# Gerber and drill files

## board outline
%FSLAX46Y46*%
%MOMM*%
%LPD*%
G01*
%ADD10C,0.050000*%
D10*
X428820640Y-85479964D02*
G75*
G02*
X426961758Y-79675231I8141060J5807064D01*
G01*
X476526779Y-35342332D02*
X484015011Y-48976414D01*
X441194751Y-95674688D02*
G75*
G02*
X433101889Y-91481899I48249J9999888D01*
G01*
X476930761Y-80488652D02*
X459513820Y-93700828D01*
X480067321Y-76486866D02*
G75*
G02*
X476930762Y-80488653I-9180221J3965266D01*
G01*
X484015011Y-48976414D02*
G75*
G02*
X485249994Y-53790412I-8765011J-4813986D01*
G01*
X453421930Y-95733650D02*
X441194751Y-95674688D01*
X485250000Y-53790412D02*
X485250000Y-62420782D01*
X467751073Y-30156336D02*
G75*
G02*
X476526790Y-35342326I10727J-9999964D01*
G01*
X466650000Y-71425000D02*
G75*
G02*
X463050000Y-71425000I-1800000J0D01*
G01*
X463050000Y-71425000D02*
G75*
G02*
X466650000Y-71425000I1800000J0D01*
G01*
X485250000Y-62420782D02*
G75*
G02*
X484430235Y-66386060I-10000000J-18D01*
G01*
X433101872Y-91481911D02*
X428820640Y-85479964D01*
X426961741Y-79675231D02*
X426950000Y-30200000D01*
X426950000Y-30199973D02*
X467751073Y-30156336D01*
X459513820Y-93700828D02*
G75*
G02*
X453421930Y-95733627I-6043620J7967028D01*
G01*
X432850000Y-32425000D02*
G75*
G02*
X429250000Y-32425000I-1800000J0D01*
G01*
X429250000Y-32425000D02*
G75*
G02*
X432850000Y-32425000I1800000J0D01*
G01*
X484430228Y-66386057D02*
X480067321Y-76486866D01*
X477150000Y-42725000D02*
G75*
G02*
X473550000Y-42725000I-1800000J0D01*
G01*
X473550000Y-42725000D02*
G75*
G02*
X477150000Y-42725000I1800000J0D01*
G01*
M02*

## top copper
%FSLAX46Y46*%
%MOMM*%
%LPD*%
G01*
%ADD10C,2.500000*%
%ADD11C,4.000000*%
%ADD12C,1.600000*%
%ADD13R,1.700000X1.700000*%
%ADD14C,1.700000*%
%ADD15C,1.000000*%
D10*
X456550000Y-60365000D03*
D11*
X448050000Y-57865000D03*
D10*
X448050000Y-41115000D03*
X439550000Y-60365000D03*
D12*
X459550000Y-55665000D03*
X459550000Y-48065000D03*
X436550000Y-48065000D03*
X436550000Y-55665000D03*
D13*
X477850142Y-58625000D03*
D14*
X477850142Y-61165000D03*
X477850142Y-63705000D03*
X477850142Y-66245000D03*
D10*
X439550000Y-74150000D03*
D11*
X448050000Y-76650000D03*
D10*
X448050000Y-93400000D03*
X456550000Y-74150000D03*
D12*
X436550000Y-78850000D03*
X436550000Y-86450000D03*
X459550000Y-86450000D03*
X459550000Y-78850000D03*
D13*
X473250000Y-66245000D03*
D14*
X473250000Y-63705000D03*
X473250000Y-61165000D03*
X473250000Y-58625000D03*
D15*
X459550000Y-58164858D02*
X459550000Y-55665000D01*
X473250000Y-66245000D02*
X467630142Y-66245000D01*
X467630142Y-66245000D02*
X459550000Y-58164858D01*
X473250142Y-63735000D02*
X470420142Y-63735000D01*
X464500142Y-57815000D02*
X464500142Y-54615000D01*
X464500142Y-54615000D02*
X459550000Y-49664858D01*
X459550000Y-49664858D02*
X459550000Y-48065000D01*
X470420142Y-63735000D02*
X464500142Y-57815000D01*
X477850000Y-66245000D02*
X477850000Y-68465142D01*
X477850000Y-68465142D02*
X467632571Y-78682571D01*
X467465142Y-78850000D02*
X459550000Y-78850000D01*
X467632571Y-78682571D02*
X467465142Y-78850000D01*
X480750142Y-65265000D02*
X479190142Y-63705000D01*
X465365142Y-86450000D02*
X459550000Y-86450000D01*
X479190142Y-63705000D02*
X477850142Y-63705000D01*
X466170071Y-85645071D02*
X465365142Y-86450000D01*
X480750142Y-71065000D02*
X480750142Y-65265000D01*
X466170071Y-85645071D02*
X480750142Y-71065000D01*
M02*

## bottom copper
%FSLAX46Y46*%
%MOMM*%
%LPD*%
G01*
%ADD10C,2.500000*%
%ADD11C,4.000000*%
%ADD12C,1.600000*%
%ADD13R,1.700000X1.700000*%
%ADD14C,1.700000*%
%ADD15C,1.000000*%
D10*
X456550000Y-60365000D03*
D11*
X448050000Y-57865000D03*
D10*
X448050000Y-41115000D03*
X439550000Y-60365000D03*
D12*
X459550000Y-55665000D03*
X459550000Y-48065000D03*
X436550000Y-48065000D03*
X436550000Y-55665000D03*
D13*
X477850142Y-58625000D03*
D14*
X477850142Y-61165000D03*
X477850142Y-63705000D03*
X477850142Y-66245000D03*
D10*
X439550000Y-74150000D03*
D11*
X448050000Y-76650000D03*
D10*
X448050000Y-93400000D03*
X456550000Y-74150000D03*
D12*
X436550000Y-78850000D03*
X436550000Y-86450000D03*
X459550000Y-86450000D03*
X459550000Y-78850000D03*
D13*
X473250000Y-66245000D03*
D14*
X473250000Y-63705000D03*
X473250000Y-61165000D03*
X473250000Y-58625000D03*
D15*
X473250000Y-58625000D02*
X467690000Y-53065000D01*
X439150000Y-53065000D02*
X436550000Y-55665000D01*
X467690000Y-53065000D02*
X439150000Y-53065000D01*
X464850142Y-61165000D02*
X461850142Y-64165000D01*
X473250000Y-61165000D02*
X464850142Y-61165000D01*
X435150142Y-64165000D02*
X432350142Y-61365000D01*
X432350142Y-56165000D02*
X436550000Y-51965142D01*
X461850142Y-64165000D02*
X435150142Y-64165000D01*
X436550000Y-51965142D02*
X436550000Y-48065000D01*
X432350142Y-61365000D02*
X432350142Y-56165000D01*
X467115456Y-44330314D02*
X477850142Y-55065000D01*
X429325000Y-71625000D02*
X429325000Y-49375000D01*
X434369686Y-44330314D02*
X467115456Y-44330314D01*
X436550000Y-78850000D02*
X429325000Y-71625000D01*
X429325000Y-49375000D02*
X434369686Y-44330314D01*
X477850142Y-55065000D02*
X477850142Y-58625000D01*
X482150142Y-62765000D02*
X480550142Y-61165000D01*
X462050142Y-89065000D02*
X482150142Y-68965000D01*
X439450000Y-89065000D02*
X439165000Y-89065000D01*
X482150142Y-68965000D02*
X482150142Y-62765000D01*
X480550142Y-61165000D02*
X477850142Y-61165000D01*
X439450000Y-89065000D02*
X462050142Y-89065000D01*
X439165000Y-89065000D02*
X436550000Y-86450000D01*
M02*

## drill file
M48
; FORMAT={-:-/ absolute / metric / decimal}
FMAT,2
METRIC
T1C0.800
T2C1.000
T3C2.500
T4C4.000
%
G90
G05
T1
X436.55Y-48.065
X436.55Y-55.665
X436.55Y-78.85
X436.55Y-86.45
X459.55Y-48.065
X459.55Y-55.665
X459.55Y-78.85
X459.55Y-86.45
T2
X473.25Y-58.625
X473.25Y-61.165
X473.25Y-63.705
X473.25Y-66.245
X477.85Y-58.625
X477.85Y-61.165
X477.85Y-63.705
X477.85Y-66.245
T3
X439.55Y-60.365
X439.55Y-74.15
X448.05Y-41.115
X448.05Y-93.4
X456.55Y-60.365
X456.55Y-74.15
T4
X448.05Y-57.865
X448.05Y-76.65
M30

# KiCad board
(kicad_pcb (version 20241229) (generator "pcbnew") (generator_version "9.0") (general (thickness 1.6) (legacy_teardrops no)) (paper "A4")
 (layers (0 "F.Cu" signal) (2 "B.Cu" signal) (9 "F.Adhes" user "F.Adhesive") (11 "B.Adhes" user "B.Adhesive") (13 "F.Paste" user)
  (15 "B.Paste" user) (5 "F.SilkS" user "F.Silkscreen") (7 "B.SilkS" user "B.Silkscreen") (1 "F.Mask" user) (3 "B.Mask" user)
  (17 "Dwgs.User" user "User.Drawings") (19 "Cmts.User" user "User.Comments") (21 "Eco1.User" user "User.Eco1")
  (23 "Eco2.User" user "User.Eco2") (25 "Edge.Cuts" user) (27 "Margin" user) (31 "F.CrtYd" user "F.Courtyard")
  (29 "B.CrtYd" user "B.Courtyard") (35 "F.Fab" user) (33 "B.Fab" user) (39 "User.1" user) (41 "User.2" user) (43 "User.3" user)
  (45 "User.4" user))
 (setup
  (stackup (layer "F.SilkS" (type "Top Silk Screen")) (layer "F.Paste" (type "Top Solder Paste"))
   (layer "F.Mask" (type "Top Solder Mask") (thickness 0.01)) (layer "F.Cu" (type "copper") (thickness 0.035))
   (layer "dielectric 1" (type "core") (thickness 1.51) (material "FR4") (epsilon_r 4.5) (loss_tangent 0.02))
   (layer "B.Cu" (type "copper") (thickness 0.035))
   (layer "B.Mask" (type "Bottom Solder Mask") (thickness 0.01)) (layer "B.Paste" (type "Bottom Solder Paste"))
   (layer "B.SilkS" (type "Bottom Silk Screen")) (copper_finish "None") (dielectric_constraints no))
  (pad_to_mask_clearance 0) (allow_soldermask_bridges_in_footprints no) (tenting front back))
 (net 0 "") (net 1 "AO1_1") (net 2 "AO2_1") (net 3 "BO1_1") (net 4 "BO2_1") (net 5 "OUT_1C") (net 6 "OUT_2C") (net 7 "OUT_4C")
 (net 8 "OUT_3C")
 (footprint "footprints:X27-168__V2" (layer "F.Cu") (at 448.05 51.865 180)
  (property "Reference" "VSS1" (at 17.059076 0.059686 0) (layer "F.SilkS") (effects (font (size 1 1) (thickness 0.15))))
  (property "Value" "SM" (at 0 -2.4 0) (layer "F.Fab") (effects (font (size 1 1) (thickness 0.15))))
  (pad "" thru_hole circle (at -8.5 -8.5 180) (size 2.5 2.5) (drill 2.5) (layers "*.Cu" "*.Mask") (remove_unused_layers no))
  (pad "" thru_hole circle (at 0 -6 180) (size 4 4) (drill 4) (layers "*.Cu" "*.Mask") (remove_unused_layers no))
  (pad "" thru_hole circle (at 0 10.75 180) (size 2.5 2.5) (drill 2.5) (layers "*.Cu" "*.Mask") (remove_unused_layers no))
  (pad "" thru_hole circle (at 8.5 -8.5 180) (size 2.5 2.5) (drill 2.5) (layers "*.Cu" "*.Mask") (remove_unused_layers no))
  (pad "1" thru_hole circle (at -11.5 -3.8 180) (size 1.6 1.6) (drill 0.8) (layers "*.Cu" "*.Mask") (remove_unused_layers no)
   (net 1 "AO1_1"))
  (pad "2" thru_hole circle (at -11.5 3.8 180) (size 1.6 1.6) (drill 0.8) (layers "*.Cu" "*.Mask") (remove_unused_layers no) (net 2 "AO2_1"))
  (pad "3" thru_hole circle (at 11.5 3.8 180) (size 1.6 1.6) (drill 0.8) (layers "*.Cu" "*.Mask") (remove_unused_layers no) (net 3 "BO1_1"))
  (pad "4" thru_hole circle (at 11.5 -3.8 180) (size 1.6 1.6) (drill 0.8) (layers "*.Cu" "*.Mask") (remove_unused_layers no) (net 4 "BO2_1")))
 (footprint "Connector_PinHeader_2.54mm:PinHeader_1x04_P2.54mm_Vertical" (layer "F.Cu") (at 477.850142 58.625)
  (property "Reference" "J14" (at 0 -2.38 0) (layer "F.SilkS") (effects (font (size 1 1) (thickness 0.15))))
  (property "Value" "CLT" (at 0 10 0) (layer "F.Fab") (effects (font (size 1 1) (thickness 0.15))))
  (pad "1" thru_hole rect (at 0 0) (size 1.7 1.7) (drill 1) (layers "*.Cu" "*.Mask") (remove_unused_layers no) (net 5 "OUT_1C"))
  (pad "2" thru_hole circle (at 0 2.54) (size 1.7 1.7) (drill 1) (layers "*.Cu" "*.Mask") (remove_unused_layers no) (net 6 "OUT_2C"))
  (pad "3" thru_hole circle (at 0 5.08) (size 1.7 1.7) (drill 1) (layers "*.Cu" "*.Mask") (remove_unused_layers no) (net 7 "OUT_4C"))
  (pad "4" thru_hole circle (at 0 7.62) (size 1.7 1.7) (drill 1) (layers "*.Cu" "*.Mask") (remove_unused_layers no) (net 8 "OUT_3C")))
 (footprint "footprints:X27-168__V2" (layer "F.Cu") (at 448.05 82.65)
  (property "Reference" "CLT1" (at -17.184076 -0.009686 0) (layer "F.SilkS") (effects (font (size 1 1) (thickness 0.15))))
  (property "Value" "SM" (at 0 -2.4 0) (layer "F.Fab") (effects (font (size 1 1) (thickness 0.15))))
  (pad "" thru_hole circle (at -8.5 -8.5) (size 2.5 2.5) (drill 2.5) (layers "*.Cu" "*.Mask") (remove_unused_layers no))
  (pad "" thru_hole circle (at 0 -6) (size 4 4) (drill 4) (layers "*.Cu" "*.Mask") (remove_unused_layers no))
  (pad "" thru_hole circle (at 0 10.75) (size 2.5 2.5) (drill 2.5) (layers "*.Cu" "*.Mask") (remove_unused_layers no))
  (pad "" thru_hole circle (at 8.5 -8.5) (size 2.5 2.5) (drill 2.5) (layers "*.Cu" "*.Mask") (remove_unused_layers no))
  (pad "1" thru_hole circle (at -11.5 -3.8) (size 1.6 1.6) (drill 0.8) (layers "*.Cu" "*.Mask") (remove_unused_layers no) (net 5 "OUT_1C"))
  (pad "2" thru_hole circle (at -11.5 3.8) (size 1.6 1.6) (drill 0.8) (layers "*.Cu" "*.Mask") (remove_unused_layers no) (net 6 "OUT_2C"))
  (pad "3" thru_hole circle (at 11.5 3.8) (size 1.6 1.6) (drill 0.8) (layers "*.Cu" "*.Mask") (remove_unused_layers no) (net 7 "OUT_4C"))
  (pad "4" thru_hole circle (at 11.5 -3.8) (size 1.6 1.6) (drill 0.8) (layers "*.Cu" "*.Mask") (remove_unused_layers no) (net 8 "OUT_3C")))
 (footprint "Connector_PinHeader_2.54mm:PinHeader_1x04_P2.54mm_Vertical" (layer "B.Cu") (at 473.25 66.245)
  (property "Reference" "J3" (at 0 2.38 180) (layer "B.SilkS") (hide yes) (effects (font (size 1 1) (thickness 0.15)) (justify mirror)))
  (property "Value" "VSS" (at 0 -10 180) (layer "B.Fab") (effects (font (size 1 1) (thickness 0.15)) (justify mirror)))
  (pad "1" thru_hole rect (at 0 0) (size 1.7 1.7) (drill 1) (layers "*.Cu" "*.Mask") (remove_unused_layers no) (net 1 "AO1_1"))
  (pad "2" thru_hole circle (at 0 -2.54) (size 1.7 1.7) (drill 1) (layers "*.Cu" "*.Mask") (remove_unused_layers no) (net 2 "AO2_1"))
  (pad "3" thru_hole circle (at 0 -5.08) (size 1.7 1.7) (drill 1) (layers "*.Cu" "*.Mask") (remove_unused_layers no) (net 3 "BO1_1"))
  (pad "4" thru_hole circle (at 0 -7.62) (size 1.7 1.7) (drill 1) (layers "*.Cu" "*.Mask") (remove_unused_layers no) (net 4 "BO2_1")))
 (gr_arc (start 428.82064 85.479964) (mid 427.438159 82.722676) (end 426.961741 79.675231) (stroke (width 0.05) (type default))
  (layer "Edge.Cuts"))
 (gr_line (start 476.526779 35.342332) (end 484.015011 48.976414) (stroke (width 0.05) (type default)) (layer "Edge.Cuts"))
 (gr_arc (start 441.194751 95.674688) (mid 436.642854 94.553932) (end 433.101872 91.481911) (stroke (width 0.05) (type default))
  (layer "Edge.Cuts"))
 (gr_line (start 476.930761 80.488652) (end 459.51382 93.700828) (stroke (width 0.05) (type default)) (layer "Edge.Cuts"))
 (gr_arc (start 480.067321 76.486866) (mid 478.757629 78.690438) (end 476.930761 80.488652) (stroke (width 0.05) (type default))
  (layer "Edge.Cuts"))
 (gr_arc (start 484.015011 48.976414) (mid 484.936333 51.305469) (end 485.25 53.790412) (stroke (width 0.05) (type default))
  (layer "Edge.Cuts"))
 (gr_line (start 453.42193 95.73365) (end 441.194751 95.674688) (stroke (width 0.05) (type default)) (layer "Edge.Cuts"))
 (gr_line (start 485.25 53.790412) (end 485.25 62.420782) (stroke (width 0.05) (type default)) (layer "Edge.Cuts"))
 (gr_arc (start 467.751073 30.156336) (mid 472.849324 31.547206) (end 476.526779 35.342332) (stroke (width 0.05) (type default))
  (layer "Edge.Cuts"))
 (gr_circle (center 464.85 71.425) (end 463.05 71.425) (stroke (width 0.05) (type default)) (fill no) (layer "Edge.Cuts"))
 (gr_arc (start 485.25 62.420782) (mid 485.042913 64.445346) (end 484.430228 66.386057) (stroke (width 0.05) (type default))
  (layer "Edge.Cuts"))
 (gr_line (start 433.101872 91.481911) (end 428.82064 85.479964) (stroke (width 0.05) (type default)) (layer "Edge.Cuts"))
 (gr_line (start 426.961741 79.675231) (end 426.95 30.2) (stroke (width 0.05) (type default)) (layer "Edge.Cuts"))
 (gr_line (start 426.95 30.199973) (end 467.751073 30.156336) (stroke (width 0.05) (type default)) (layer "Edge.Cuts"))
 (gr_arc (start 459.51382 93.700828) (mid 456.635501 95.219575) (end 453.42193 95.73365) (stroke (width 0.05) (type default))
  (layer "Edge.Cuts"))
 (gr_circle (center 431.05 32.425) (end 429.25 32.425) (stroke (width 0.05) (type default)) (fill no) (layer "Edge.Cuts"))
 (gr_line (start 484.430228 66.386057) (end 480.067321 76.486866) (stroke (width 0.05) (type default)) (layer "Edge.Cuts"))
 (gr_circle (center 475.35 42.725) (end 473.55 42.725) (stroke (width 0.05) (type default)) (fill no) (layer "Edge.Cuts"))
 (segment (start 459.55 58.164858) (end 459.55 55.665) (width 1) (layer "F.Cu") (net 1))
 (segment (start 473.25 66.245) (end 467.630142 66.245) (width 1) (layer "F.Cu") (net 1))
 (segment (start 467.630142 66.245) (end 459.55 58.164858) (width 1) (layer "F.Cu") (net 1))
 (segment (start 473.25 58.625) (end 467.69 53.065) (width 1) (layer "B.Cu") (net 4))
 (segment (start 439.15 53.065) (end 436.55 55.665) (width 1) (layer "B.Cu") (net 4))
 (segment (start 467.69 53.065) (end 439.15 53.065) (width 1) (layer "B.Cu") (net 4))
 (segment (start 464.850142 61.165) (end 461.850142 64.165) (width 1) (layer "B.Cu") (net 3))
 (segment (start 473.25 61.165) (end 464.850142 61.165) (width 1) (layer "B.Cu") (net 3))
 (segment (start 435.150142 64.165) (end 432.350142 61.365) (width 1) (layer "B.Cu") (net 3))
 (segment (start 432.350142 56.165) (end 436.55 51.965142) (width 1) (layer "B.Cu") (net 3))
 (segment (start 461.850142 64.165) (end 435.150142 64.165) (width 1) (layer "B.Cu") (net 3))
 (segment (start 436.55 51.965142) (end 436.55 48.065) (width 1) (layer "B.Cu") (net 3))
 (segment (start 432.350142 61.365) (end 432.350142 56.165) (width 1) (layer "B.Cu") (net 3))
 (segment (start 473.250142 63.735) (end 470.420142 63.735) (width 1) (layer "F.Cu") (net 2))
 (segment (start 464.500142 57.815) (end 464.500142 54.615) (width 1) (layer "F.Cu") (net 2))
 (segment (start 464.500142 54.615) (end 459.55 49.664858) (width 1) (layer "F.Cu") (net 2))
 (segment (start 459.55 49.664858) (end 459.55 48.065) (width 1) (layer "F.Cu") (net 2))
 (segment (start 470.420142 63.735) (end 464.500142 57.815) (width 1) (layer "F.Cu") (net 2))
 (segment (start 477.85 66.245) (end 477.85 68.465142) (width 1) (layer "F.Cu") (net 8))
 (segment (start 477.85 68.465142) (end 467.632571 78.682571) (width 1) (layer "F.Cu") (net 8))
 (segment (start 467.465142 78.85) (end 459.55 78.85) (width 1) (layer "F.Cu") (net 8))
 (segment (start 467.632571 78.682571) (end 467.465142 78.85) (width 1) (layer "F.Cu") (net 8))
 (segment (start 467.115456 44.330314) (end 477.850142 55.065) (width 1) (layer "B.Cu") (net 5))
 (segment (start 429.325 71.625) (end 429.325 49.375) (width 1) (layer "B.Cu") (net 5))
 (segment (start 434.369686 44.330314) (end 467.115456 44.330314) (width 1) (layer "B.Cu") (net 5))
 (segment (start 436.55 78.85) (end 429.325 71.625) (width 1) (layer "B.Cu") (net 5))
 (segment (start 429.325 49.375) (end 434.369686 44.330314) (width 1) (layer "B.Cu") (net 5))
 (segment (start 477.850142 55.065) (end 477.850142 58.625) (width 1) (layer "B.Cu") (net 5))
 (segment (start 480.750142 65.265) (end 479.190142 63.705) (width 1) (layer "F.Cu") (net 7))
 (segment (start 465.365142 86.45) (end 459.55 86.45) (width 1) (layer "F.Cu") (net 7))
 (segment (start 479.190142 63.705) (end 477.850142 63.705) (width 1) (layer "F.Cu") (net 7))
 (segment (start 466.170071 85.645071) (end 465.365142 86.45) (width 1) (layer "F.Cu") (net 7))
 (segment (start 480.750142 71.065) (end 480.750142 65.265) (width 1) (layer "F.Cu") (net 7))
 (segment (start 466.170071 85.645071) (end 480.750142 71.065) (width 1) (layer "F.Cu") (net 7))
 (segment (start 482.150142 62.765) (end 480.550142 61.165) (width 1) (layer "B.Cu") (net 6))
 (segment (start 462.050142 89.065) (end 482.150142 68.965) (width 1) (layer "B.Cu") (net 6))
 (segment (start 439.45 89.065) (end 439.165 89.065) (width 1) (layer "B.Cu") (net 6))
 (segment (start 482.150142 68.965) (end 482.150142 62.765) (width 1) (layer "B.Cu") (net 6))
 (segment (start 480.550142 61.165) (end 477.850142 61.165) (width 1) (layer "B.Cu") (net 6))
 (segment (start 439.45 89.065) (end 462.050142 89.065) (width 1) (layer "B.Cu") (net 6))
 (segment (start 439.165 89.065) (end 436.55 86.45) (width 1) (layer "B.Cu") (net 6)))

